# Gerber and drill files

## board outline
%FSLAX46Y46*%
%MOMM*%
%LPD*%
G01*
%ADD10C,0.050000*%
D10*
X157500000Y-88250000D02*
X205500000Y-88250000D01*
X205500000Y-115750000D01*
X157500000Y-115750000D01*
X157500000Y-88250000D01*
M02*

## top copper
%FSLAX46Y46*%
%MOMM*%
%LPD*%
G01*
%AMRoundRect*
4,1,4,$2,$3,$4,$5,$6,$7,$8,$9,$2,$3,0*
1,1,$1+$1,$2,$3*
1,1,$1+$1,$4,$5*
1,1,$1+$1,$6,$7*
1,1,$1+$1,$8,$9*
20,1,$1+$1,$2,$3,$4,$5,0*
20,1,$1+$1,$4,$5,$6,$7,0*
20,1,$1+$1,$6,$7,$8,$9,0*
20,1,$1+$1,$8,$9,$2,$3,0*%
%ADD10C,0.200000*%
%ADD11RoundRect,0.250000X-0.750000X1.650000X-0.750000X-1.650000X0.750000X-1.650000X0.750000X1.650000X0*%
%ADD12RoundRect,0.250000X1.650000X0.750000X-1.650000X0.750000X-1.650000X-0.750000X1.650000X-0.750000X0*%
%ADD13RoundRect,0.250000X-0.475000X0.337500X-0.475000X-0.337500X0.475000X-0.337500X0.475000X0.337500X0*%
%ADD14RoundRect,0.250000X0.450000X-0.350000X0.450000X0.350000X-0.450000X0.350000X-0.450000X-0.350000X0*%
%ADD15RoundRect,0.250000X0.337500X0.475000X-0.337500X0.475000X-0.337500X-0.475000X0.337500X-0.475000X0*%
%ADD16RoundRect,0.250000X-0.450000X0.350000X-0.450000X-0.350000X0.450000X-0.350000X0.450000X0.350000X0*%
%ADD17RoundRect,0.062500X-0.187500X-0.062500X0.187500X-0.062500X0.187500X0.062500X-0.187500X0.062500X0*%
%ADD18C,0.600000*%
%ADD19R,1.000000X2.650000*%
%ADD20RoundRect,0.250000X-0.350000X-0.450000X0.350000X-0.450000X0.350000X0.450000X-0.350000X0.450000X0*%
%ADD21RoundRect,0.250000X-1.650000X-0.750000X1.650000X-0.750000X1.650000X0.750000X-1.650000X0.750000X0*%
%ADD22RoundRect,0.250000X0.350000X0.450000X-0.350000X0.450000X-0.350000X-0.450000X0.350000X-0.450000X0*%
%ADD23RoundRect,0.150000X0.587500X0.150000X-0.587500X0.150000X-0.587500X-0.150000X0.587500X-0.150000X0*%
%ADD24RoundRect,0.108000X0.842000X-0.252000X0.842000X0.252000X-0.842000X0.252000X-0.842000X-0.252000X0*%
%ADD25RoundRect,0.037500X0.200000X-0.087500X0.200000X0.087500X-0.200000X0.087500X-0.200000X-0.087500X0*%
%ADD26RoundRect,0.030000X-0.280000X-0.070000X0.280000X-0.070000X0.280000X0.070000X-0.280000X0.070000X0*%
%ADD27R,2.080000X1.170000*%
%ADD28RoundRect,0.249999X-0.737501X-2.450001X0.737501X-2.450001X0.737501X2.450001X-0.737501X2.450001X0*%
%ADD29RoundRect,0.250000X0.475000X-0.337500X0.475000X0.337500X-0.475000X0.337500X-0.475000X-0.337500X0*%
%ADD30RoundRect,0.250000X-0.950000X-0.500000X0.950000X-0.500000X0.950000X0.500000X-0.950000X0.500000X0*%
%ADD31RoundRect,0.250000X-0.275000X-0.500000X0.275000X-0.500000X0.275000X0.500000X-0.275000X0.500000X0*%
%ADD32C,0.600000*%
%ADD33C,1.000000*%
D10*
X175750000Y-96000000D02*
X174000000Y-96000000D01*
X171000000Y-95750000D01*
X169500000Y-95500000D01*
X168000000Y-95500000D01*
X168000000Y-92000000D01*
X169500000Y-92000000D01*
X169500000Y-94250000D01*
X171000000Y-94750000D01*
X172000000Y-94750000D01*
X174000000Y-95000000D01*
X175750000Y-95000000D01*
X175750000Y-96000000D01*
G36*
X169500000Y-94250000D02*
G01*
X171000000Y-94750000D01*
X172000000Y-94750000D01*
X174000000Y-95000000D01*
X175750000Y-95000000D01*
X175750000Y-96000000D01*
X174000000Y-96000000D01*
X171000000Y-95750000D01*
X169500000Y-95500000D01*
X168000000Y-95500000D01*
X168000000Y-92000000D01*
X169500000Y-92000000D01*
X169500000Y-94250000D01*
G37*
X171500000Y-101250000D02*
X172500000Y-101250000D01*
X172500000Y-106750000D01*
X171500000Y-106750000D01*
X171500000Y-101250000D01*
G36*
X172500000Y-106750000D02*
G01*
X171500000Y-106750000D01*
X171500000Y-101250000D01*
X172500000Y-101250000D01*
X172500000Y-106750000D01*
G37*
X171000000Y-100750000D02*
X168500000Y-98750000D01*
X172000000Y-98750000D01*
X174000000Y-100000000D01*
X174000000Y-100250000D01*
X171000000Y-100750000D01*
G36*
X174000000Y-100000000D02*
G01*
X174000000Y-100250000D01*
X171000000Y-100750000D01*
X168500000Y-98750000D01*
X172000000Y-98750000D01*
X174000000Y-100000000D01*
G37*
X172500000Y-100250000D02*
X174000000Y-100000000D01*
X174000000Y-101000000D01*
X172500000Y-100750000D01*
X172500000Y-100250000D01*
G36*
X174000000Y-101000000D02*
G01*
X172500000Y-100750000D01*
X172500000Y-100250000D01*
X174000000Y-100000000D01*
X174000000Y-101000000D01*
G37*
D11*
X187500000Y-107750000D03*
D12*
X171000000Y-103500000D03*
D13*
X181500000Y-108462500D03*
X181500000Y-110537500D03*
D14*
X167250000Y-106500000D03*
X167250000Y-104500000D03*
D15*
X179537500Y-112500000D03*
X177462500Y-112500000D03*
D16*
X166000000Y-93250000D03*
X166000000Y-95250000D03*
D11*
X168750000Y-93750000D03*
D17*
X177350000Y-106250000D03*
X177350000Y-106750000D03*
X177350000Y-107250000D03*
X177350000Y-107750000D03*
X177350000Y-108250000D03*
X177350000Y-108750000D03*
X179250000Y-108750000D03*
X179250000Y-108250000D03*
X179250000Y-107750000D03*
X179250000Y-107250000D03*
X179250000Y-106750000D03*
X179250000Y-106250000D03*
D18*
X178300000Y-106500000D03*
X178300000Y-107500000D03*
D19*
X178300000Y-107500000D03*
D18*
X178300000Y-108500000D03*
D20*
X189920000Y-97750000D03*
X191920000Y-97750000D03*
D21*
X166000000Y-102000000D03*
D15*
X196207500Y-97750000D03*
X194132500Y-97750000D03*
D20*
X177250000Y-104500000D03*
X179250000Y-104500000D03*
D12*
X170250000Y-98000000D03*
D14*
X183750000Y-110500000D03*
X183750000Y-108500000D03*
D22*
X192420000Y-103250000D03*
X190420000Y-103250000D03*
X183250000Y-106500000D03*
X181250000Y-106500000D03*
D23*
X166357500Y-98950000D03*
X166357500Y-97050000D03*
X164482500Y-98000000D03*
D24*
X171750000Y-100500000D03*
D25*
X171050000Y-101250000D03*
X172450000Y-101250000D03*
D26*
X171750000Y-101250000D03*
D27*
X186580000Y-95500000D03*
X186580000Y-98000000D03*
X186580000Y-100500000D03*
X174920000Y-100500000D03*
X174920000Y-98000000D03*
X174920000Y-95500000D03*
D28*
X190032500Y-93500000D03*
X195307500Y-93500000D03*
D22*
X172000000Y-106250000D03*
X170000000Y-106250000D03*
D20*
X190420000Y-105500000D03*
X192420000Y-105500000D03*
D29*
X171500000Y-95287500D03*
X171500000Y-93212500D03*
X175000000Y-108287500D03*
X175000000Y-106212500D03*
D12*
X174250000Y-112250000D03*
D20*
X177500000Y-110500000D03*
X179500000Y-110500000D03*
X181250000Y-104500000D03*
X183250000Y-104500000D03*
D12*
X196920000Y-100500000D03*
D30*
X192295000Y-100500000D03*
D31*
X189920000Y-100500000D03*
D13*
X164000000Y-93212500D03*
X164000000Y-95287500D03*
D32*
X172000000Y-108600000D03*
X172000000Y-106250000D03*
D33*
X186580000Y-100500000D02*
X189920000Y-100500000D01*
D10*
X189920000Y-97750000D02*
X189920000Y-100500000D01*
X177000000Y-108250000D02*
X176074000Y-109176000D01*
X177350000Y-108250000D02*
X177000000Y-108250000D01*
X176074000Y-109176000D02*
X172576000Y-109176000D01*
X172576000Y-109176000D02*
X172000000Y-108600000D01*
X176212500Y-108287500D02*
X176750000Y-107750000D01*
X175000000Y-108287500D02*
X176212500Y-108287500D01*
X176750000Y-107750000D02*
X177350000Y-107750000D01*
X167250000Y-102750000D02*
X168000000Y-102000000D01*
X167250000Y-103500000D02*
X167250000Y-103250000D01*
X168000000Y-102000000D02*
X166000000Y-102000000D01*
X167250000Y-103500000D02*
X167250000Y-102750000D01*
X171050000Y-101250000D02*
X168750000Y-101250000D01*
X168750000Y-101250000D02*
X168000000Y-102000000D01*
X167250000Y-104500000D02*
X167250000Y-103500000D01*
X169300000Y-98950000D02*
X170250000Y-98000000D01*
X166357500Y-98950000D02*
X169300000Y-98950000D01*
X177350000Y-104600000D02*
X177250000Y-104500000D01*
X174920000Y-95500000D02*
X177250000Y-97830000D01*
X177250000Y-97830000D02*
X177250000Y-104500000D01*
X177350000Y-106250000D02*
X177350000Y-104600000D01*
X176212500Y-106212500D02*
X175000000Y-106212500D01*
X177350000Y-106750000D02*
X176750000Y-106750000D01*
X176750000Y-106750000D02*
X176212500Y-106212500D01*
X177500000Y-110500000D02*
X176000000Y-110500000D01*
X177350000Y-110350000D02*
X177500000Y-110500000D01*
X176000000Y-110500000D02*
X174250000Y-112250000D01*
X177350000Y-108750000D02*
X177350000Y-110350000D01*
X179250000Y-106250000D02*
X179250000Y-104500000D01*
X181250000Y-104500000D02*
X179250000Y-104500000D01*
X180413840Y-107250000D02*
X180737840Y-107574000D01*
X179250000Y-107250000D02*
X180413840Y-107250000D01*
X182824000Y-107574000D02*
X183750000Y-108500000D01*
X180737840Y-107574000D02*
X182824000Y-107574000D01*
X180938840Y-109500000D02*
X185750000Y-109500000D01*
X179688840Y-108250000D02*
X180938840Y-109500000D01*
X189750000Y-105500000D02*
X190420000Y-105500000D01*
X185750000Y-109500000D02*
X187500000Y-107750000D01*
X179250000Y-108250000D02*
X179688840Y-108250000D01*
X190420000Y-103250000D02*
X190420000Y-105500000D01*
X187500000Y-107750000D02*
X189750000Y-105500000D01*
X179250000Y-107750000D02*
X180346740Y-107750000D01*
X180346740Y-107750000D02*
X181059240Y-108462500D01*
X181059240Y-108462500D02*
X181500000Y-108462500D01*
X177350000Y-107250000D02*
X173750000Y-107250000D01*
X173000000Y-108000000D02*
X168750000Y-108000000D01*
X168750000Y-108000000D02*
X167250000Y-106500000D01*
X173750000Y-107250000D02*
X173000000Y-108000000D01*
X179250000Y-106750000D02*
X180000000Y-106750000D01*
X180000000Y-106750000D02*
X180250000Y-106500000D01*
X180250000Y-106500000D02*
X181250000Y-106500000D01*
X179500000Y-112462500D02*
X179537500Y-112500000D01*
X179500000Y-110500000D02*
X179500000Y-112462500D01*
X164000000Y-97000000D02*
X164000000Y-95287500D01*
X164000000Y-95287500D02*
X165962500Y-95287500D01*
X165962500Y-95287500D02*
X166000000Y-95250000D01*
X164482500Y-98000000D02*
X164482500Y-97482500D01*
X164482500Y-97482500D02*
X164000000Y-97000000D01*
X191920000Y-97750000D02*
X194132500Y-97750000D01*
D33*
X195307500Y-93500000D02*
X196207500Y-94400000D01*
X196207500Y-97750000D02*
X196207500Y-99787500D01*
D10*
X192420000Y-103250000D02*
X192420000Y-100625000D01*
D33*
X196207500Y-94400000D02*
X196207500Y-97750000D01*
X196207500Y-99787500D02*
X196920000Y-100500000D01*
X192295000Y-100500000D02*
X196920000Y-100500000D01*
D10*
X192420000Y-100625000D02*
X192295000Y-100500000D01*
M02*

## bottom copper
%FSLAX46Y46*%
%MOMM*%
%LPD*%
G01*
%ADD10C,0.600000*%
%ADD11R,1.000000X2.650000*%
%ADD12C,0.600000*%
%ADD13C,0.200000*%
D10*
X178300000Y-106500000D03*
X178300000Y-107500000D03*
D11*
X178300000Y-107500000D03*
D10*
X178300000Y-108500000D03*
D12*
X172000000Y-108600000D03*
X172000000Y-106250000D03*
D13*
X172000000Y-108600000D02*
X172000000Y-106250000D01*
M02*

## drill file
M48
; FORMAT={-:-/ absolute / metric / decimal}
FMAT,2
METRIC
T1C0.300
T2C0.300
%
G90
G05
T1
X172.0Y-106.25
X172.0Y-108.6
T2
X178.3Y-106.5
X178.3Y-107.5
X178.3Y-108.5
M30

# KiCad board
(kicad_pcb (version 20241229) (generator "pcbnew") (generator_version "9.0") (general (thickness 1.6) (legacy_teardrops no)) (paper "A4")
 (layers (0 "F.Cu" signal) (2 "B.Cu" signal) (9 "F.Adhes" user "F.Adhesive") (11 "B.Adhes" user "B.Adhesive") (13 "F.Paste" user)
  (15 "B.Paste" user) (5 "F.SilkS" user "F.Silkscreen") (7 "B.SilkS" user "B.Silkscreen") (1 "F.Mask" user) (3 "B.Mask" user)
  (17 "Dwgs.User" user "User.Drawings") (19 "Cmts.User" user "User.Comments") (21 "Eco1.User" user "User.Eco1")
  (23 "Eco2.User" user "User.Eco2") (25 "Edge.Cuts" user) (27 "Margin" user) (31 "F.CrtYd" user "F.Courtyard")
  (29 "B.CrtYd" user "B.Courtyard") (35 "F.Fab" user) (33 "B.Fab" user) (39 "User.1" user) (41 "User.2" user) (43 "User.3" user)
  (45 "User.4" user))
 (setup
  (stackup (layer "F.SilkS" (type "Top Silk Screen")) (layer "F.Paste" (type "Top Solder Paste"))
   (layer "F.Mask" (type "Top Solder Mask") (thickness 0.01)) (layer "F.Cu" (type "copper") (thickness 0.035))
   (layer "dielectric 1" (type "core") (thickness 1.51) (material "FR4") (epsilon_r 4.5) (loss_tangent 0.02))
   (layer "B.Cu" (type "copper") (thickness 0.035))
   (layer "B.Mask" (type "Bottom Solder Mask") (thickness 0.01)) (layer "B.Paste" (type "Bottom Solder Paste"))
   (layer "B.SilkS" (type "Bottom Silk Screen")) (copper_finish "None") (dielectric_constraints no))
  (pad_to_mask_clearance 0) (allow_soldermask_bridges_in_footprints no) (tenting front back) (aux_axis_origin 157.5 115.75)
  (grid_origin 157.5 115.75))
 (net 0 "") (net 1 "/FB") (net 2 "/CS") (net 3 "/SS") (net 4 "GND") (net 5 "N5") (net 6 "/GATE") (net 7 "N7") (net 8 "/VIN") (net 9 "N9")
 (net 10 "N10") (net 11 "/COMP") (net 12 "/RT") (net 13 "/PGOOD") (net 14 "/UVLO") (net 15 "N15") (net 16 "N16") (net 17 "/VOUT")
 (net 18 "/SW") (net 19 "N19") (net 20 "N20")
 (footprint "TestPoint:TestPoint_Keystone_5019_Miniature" (layer "F.Cu") (at 187.5 107.75 -90)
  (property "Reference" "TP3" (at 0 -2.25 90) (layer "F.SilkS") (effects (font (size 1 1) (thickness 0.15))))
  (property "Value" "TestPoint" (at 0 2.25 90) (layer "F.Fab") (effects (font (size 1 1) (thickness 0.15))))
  (pad "1" smd roundrect (at 0 0 270) (size 3.8 2) (layers "F.Cu" "F.Mask" "F.Paste") (roundrect_rratio 0.125) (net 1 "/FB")))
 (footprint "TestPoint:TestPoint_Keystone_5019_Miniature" (layer "F.Cu") (at 171 103.5 180)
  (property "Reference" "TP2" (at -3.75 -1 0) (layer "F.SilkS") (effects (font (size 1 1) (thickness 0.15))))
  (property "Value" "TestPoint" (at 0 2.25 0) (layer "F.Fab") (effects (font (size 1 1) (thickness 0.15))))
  (pad "1" smd roundrect (at 0 0 180) (size 3.8 2) (layers "F.Cu" "F.Mask" "F.Paste") (roundrect_rratio 0.125) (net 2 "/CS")))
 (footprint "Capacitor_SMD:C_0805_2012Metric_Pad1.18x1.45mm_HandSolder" (layer "F.Cu") (at 181.5 109.5 -90)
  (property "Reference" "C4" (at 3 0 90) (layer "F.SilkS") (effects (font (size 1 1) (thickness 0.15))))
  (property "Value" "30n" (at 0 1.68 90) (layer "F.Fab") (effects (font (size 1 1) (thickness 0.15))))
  (pad "1" smd roundrect (at -1.0375 0 270) (size 1.175 1.45) (layers "F.Cu" "F.Mask" "F.Paste") (roundrect_rratio 0.212766) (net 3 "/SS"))
  (pad "2" smd roundrect (at 1.0375 0 270) (size 1.175 1.45) (layers "F.Cu" "F.Mask" "F.Paste") (roundrect_rratio 0.212766) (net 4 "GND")))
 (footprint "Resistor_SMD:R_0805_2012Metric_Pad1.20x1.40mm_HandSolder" (layer "F.Cu") (at 167.25 105.5 90)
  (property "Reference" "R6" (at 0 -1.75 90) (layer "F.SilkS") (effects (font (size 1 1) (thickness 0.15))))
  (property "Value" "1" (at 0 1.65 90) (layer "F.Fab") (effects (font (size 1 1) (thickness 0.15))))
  (pad "1" smd roundrect (at -1 0 90) (size 1.2 1.4) (layers "F.Cu" "F.Mask" "F.Paste") (roundrect_rratio 0.208333) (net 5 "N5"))
  (pad "2" smd roundrect (at 1 0 90) (size 1.2 1.4) (layers "F.Cu" "F.Mask" "F.Paste") (roundrect_rratio 0.208333) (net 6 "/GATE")))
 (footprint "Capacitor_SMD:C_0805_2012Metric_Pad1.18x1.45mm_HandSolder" (layer "F.Cu") (at 178.5 112.5 180)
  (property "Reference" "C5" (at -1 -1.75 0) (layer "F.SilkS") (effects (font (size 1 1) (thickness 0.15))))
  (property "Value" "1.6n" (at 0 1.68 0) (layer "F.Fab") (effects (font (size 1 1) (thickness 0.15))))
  (pad "1" smd roundrect (at -1.0375 0 180) (size 1.175 1.45) (layers "F.Cu" "F.Mask" "F.Paste") (roundrect_rratio 0.212766) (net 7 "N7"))
  (pad "2" smd roundrect (at 1.0375 0 180) (size 1.175 1.45) (layers "F.Cu" "F.Mask" "F.Paste") (roundrect_rratio 0.212766) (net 4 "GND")))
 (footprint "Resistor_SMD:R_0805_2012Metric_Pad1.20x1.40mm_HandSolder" (layer "F.Cu") (at 166 94.25 -90)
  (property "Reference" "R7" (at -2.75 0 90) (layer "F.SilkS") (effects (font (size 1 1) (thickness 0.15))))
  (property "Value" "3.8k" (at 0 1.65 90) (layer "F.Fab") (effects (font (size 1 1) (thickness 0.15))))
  (pad "1" smd roundrect (at -1 0 270) (size 1.2 1.4) (layers "F.Cu" "F.Mask" "F.Paste") (roundrect_rratio 0.208333) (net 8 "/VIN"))
  (pad "2" smd roundrect (at 1 0 270) (size 1.2 1.4) (layers "F.Cu" "F.Mask" "F.Paste") (roundrect_rratio 0.208333) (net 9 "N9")))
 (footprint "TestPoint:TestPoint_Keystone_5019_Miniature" (layer "F.Cu") (at 168.75 93.75 -90)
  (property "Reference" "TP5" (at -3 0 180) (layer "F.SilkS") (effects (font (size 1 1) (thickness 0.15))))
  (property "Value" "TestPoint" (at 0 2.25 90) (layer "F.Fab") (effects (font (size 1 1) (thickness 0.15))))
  (pad "1" smd roundrect (at 0 0 270) (size 3.8 2) (layers "F.Cu" "F.Mask" "F.Paste") (roundrect_rratio 0.125) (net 8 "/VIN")))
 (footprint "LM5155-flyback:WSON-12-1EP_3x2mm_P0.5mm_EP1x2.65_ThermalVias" (layer "F.Cu") (at 178.3 107.5)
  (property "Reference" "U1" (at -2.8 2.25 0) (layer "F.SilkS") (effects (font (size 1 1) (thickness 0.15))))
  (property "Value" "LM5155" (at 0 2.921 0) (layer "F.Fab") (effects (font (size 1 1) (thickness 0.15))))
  (pad "" smd rect (at 0 -0.5) (size 0.95 0.8) (layers "F.Paste"))
  (pad "" smd rect (at 0 0.5) (size 0.95 0.8) (layers "F.Paste"))
  (pad "1" smd roundrect (at -0.95 -1.25) (size 0.5 0.25) (layers "F.Cu" "F.Mask" "F.Paste") (roundrect_rratio 0.25) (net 8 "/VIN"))
  (pad "2" smd roundrect (at -0.95 -0.75) (size 0.5 0.25) (layers "F.Cu" "F.Mask" "F.Paste") (roundrect_rratio 0.25) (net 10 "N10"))
  (pad "3" smd roundrect (at -0.95 -0.25) (size 0.5 0.25) (layers "F.Cu" "F.Mask" "F.Paste") (roundrect_rratio 0.25) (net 5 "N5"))
  (pad "4" smd roundrect (at -0.95 0.25) (size 0.5 0.25) (layers "F.Cu" "F.Mask" "F.Paste") (roundrect_rratio 0.25) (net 4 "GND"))
  (pad "5" smd roundrect (at -0.95 0.75) (size 0.5 0.25) (layers "F.Cu" "F.Mask" "F.Paste") (roundrect_rratio 0.25) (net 2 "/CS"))
  (pad "6" smd roundrect (at -0.95 1.25) (size 0.5 0.25) (layers "F.Cu" "F.Mask" "F.Paste") (roundrect_rratio 0.25) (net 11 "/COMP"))
  (pad "7" smd roundrect (at 0.95 1.25) (size 0.5 0.25) (layers "F.Cu" "F.Mask" "F.Paste") (roundrect_rratio 0.25) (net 4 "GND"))
  (pad "8" smd roundrect (at 0.95 0.75) (size 0.5 0.25) (layers "F.Cu" "F.Mask" "F.Paste") (roundrect_rratio 0.25) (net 1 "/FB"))
  (pad "9" smd roundrect (at 0.95 0.25) (size 0.5 0.25) (layers "F.Cu" "F.Mask" "F.Paste") (roundrect_rratio 0.25) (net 3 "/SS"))
  (pad "10" smd roundrect (at 0.95 -0.25) (size 0.5 0.25) (layers "F.Cu" "F.Mask" "F.Paste") (roundrect_rratio 0.25) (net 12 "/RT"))
  (pad "11" smd roundrect (at 0.95 -0.75) (size 0.5 0.25) (layers "F.Cu" "F.Mask" "F.Paste") (roundrect_rratio 0.25) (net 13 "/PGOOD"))
  (pad "12" smd roundrect (at 0.95 -1.25) (size 0.5 0.25) (layers "F.Cu" "F.Mask" "F.Paste") (roundrect_rratio 0.25) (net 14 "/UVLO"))
  (pad "13" thru_hole circle (at 0 -1 90) (size 0.6 0.6) (drill 0.3) (layers "*.Cu") (remove_unused_layers no) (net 4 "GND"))
  (pad "13" thru_hole circle (at 0 0) (size 0.6 0.6) (drill 0.3) (layers "*.Cu") (remove_unused_layers no) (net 4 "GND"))
  (pad "13" smd rect (at 0 0) (size 1 2.65) (layers "F.Cu" "F.Mask") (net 4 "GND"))
  (pad "13" smd rect (at 0 0) (size 1 2.65) (layers "B.Cu") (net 4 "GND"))
  (pad "13" thru_hole circle (at 0 1) (size 0.6 0.6) (drill 0.3) (layers "*.Cu") (remove_unused_layers no) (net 4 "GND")))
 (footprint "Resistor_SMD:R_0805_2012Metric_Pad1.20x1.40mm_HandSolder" (layer "F.Cu") (at 190.92 97.75)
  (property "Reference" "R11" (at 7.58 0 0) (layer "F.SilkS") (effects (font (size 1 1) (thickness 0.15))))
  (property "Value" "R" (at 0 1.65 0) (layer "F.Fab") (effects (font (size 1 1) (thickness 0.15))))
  (pad "1" smd roundrect (at -1 0) (size 1.2 1.4) (layers "F.Cu" "F.Mask" "F.Paste") (roundrect_rratio 0.208333) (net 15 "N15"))
  (pad "2" smd roundrect (at 1 0) (size 1.2 1.4) (layers "F.Cu" "F.Mask" "F.Paste") (roundrect_rratio 0.208333) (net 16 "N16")))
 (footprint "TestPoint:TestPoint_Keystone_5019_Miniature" (layer "F.Cu") (at 166 102)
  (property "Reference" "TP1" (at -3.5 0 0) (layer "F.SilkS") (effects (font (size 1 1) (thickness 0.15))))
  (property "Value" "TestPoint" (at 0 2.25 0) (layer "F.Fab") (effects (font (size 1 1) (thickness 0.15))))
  (pad "1" smd roundrect (at 0 0) (size 3.8 2) (layers "F.Cu" "F.Mask" "F.Paste") (roundrect_rratio 0.125) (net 6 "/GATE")))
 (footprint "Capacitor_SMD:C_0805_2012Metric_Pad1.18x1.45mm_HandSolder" (layer "F.Cu") (at 195.17 97.75 180)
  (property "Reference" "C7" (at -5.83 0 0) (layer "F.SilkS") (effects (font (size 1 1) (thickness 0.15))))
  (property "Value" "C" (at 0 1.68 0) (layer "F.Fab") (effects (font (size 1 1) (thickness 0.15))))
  (pad "1" smd roundrect (at -1.0375 0 180) (size 1.175 1.45) (layers "F.Cu" "F.Mask" "F.Paste") (roundrect_rratio 0.212766)
   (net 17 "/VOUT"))
  (pad "2" smd roundrect (at 1.0375 0 180) (size 1.175 1.45) (layers "F.Cu" "F.Mask" "F.Paste") (roundrect_rratio 0.212766) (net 16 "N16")))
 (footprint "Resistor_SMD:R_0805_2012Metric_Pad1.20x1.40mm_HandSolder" (layer "F.Cu") (at 178.25 104.5)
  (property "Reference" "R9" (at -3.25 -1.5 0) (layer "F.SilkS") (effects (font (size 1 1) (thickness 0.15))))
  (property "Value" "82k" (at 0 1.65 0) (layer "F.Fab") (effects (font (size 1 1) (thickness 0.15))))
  (pad "1" smd roundrect (at -1 0) (size 1.2 1.4) (layers "F.Cu" "F.Mask" "F.Paste") (roundrect_rratio 0.208333) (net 8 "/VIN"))
  (pad "2" smd roundrect (at 1 0) (size 1.2 1.4) (layers "F.Cu" "F.Mask" "F.Paste") (roundrect_rratio 0.208333) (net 14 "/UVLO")))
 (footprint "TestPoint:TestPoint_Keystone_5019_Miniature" (layer "F.Cu") (at 170.25 98 180)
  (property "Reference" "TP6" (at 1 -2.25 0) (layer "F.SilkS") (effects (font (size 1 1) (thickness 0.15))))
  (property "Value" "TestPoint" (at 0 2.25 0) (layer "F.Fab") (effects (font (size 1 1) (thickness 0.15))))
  (pad "1" smd roundrect (at 0 0 180) (size 3.8 2) (layers "F.Cu" "F.Mask" "F.Paste") (roundrect_rratio 0.125) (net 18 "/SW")))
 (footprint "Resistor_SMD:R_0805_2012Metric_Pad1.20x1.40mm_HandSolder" (layer "F.Cu") (at 183.75 109.5 90)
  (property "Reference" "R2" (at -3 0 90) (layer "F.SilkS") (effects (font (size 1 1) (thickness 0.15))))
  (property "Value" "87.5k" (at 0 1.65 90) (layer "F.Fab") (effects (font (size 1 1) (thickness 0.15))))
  (pad "1" smd roundrect (at -1 0 90) (size 1.2 1.4) (layers "F.Cu" "F.Mask" "F.Paste") (roundrect_rratio 0.208333) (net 4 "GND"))
  (pad "2" smd roundrect (at 1 0 90) (size 1.2 1.4) (layers "F.Cu" "F.Mask" "F.Paste") (roundrect_rratio 0.208333) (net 12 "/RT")))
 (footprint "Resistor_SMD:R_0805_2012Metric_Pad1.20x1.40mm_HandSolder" (layer "F.Cu") (at 191.42 103.25 180)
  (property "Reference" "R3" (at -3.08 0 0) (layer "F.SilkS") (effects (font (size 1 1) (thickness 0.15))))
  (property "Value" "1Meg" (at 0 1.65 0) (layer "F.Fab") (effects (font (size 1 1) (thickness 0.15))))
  (pad "1" smd roundrect (at -1 0 180) (size 1.2 1.4) (layers "F.Cu" "F.Mask" "F.Paste") (roundrect_rratio 0.208333) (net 17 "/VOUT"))
  (pad "2" smd roundrect (at 1 0 180) (size 1.2 1.4) (layers "F.Cu" "F.Mask" "F.Paste") (roundrect_rratio 0.208333) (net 1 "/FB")))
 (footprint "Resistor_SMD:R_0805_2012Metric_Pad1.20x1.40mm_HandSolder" (layer "F.Cu") (at 182.25 106.5 180)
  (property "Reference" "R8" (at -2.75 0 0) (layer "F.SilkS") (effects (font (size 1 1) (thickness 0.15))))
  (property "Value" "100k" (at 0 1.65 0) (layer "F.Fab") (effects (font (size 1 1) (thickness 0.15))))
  (pad "1" smd roundrect (at -1 0 180) (size 1.2 1.4) (layers "F.Cu" "F.Mask" "F.Paste") (roundrect_rratio 0.208333) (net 8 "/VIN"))
  (pad "2" smd roundrect (at 1 0 180) (size 1.2 1.4) (layers "F.Cu" "F.Mask" "F.Paste") (roundrect_rratio 0.208333) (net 13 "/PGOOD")))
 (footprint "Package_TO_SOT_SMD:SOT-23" (layer "F.Cu") (at 165.42 98 180)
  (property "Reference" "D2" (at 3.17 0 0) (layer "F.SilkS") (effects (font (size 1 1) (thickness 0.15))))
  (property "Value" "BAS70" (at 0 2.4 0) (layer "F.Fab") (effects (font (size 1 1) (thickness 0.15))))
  (pad "1" smd roundrect (at -0.9375 -0.95 180) (size 1.475 0.6) (layers "F.Cu" "F.Mask" "F.Paste") (roundrect_rratio 0.25) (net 18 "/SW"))
  (pad "2" smd roundrect (at -0.9375 0.95 180) (size 1.475 0.6) (layers "F.Cu" "F.Mask" "F.Paste") (roundrect_rratio 0.25) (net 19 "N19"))
  (pad "3" smd roundrect (at 0.9375 0 180) (size 1.475 0.6) (layers "F.Cu" "F.Mask" "F.Paste") (roundrect_rratio 0.25) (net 9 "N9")))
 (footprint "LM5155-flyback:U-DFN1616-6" (layer "F.Cu") (at 171.75 100.75 -90)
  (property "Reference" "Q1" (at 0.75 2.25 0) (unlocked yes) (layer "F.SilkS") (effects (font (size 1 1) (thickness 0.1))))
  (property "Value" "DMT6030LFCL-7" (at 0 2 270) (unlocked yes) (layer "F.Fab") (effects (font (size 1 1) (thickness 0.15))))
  (pad "1" smd roundrect (at -0.25 0 90) (size 0.72 1.9) (layers "F.Cu" "F.Mask" "F.Paste") (roundrect_rratio 0.15) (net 18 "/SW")
   (thermal_bridge_angle 45))
  (pad "2" smd roundrect (at 0.5 0.7 90) (size 0.25 0.475) (layers "F.Cu" "F.Mask" "F.Paste") (roundrect_rratio 0.15) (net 6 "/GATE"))
  (pad "3" smd roundrect (at 0.5 -0.7 90) (size 0.25 0.475) (layers "F.Cu" "F.Mask" "F.Paste") (roundrect_rratio 0.15) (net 2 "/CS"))
  (pad "3" smd roundrect (at 0.5 0) (size 0.62 0.2) (layers "F.Cu" "F.Mask" "F.Paste") (roundrect_rratio 0.15) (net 2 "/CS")))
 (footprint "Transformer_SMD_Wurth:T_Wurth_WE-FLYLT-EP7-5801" (layer "F.Cu") (at 180.75 98 -90)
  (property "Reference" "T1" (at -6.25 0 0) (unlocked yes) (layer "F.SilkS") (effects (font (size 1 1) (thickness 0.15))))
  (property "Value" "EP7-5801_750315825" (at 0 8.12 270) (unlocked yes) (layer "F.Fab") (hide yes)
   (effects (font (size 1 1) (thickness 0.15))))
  (pad "1" smd rect (at -2.5 -5.83 270) (size 1.17 2.08) (layers "F.Cu" "F.Mask" "F.Paste") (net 4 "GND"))
  (pad "2" smd rect (at 0 -5.83 270) (size 1.17 2.08) (layers "F.Cu" "F.Mask" "F.Paste") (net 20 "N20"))
  (pad "3" smd rect (at 2.5 -5.83 270) (size 1.17 2.08) (layers "F.Cu" "F.Mask" "F.Paste") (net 15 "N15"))
  (pad "4" smd rect (at 2.5 5.83 270) (size 1.17 2.08) (layers "F.Cu" "F.Mask" "F.Paste") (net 18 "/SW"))
  (pad "5" smd rect (at 0 5.83 270) (size 1.17 2.08) (layers "F.Cu" "F.Mask" "F.Paste"))
  (pad "6" smd rect (at -2.5 5.83 270) (size 1.17 2.08) (layers "F.Cu" "F.Mask" "F.Paste") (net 8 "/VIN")))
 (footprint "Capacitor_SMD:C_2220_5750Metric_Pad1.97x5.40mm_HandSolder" (layer "F.Cu") (at 192.67 93.5)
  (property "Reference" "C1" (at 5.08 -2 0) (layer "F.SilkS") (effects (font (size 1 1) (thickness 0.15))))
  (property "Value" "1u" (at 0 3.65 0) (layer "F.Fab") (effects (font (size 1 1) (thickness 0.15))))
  (pad "1" smd roundrect (at -2.6375 0) (size 1.975 5.4) (layers "F.Cu" "F.Mask" "F.Paste") (roundrect_rratio 0.126582) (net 4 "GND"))
  (pad "2" smd roundrect (at 2.6375 0) (size 1.975 5.4) (layers "F.Cu" "F.Mask" "F.Paste") (roundrect_rratio 0.126582) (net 17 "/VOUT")))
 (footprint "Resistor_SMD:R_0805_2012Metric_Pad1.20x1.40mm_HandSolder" (layer "F.Cu") (at 171 106.25 180)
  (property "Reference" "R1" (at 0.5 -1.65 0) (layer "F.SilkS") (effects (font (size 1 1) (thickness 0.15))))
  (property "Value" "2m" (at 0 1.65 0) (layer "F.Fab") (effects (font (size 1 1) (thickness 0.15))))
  (pad "1" smd roundrect (at -1 0 180) (size 1.2 1.4) (layers "F.Cu" "F.Mask" "F.Paste") (roundrect_rratio 0.208333) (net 2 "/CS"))
  (pad "2" smd roundrect (at 1 0 180) (size 1.2 1.4) (layers "F.Cu" "F.Mask" "F.Paste") (roundrect_rratio 0.208333) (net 4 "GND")))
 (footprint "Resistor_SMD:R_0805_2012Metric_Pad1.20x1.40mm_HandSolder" (layer "F.Cu") (at 191.42 105.5)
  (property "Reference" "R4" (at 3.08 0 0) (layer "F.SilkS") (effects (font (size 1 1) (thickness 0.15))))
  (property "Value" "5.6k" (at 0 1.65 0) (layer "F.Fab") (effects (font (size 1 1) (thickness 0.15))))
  (pad "1" smd roundrect (at -1 0) (size 1.2 1.4) (layers "F.Cu" "F.Mask" "F.Paste") (roundrect_rratio 0.208333) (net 1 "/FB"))
  (pad "2" smd roundrect (at 1 0) (size 1.2 1.4) (layers "F.Cu" "F.Mask" "F.Paste") (roundrect_rratio 0.208333) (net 4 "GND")))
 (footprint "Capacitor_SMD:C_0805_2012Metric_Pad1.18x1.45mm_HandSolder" (layer "F.Cu") (at 171.5 94.25 90)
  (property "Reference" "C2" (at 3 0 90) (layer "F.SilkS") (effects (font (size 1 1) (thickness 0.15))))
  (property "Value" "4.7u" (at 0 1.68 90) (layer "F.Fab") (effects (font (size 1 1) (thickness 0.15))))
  (pad "1" smd roundrect (at -1.0375 0 90) (size 1.175 1.45) (layers "F.Cu" "F.Mask" "F.Paste") (roundrect_rratio 0.212766) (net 8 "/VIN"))
  (pad "2" smd roundrect (at 1.0375 0 90) (size 1.175 1.45) (layers "F.Cu" "F.Mask" "F.Paste") (roundrect_rratio 0.212766) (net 4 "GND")))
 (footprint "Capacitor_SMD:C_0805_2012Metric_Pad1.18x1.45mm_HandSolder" (layer "F.Cu") (at 175 107.25 90)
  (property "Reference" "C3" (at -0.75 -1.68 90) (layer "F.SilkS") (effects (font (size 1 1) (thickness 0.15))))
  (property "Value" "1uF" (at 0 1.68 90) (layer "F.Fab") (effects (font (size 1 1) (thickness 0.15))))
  (pad "1" smd roundrect (at -1.0375 0 90) (size 1.175 1.45) (layers "F.Cu" "F.Mask" "F.Paste") (roundrect_rratio 0.212766) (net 4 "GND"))
  (pad "2" smd roundrect (at 1.0375 0 90) (size 1.175 1.45) (layers "F.Cu" "F.Mask" "F.Paste") (roundrect_rratio 0.212766) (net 10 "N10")))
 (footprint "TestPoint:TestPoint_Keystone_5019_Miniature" (layer "F.Cu") (at 174.25 112.25 180)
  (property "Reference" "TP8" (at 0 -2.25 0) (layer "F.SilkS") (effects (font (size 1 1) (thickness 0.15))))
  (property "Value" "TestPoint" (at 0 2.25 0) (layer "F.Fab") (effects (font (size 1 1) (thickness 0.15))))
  (pad "1" smd roundrect (at 0 0 180) (size 3.8 2) (layers "F.Cu" "F.Mask" "F.Paste") (roundrect_rratio 0.125) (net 11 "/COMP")))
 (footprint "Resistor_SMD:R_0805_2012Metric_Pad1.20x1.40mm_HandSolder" (layer "F.Cu") (at 178.5 110.5)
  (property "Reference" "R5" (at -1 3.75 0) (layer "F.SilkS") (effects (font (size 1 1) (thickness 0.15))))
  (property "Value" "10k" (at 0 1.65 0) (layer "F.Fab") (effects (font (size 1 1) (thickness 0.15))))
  (pad "1" smd roundrect (at -1 0) (size 1.2 1.4) (layers "F.Cu" "F.Mask" "F.Paste") (roundrect_rratio 0.208333) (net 11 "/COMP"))
  (pad "2" smd roundrect (at 1 0) (size 1.2 1.4) (layers "F.Cu" "F.Mask" "F.Paste") (roundrect_rratio 0.208333) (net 7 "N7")))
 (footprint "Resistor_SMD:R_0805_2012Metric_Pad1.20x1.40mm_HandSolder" (layer "F.Cu") (at 182.25 104.5)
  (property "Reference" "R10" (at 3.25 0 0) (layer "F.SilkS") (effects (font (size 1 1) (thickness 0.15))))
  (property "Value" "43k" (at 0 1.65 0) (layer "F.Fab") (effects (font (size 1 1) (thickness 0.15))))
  (pad "1" smd roundrect (at -1 0) (size 1.2 1.4) (layers "F.Cu" "F.Mask" "F.Paste") (roundrect_rratio 0.208333) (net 14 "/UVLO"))
  (pad "2" smd roundrect (at 1 0) (size 1.2 1.4) (layers "F.Cu" "F.Mask" "F.Paste") (roundrect_rratio 0.208333) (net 4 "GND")))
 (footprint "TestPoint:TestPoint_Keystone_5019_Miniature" (layer "F.Cu") (at 196.92 100.5 180)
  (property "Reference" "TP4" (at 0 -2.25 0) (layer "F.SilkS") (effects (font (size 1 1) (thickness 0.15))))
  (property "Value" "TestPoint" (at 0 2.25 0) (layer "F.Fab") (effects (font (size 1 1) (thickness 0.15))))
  (pad "1" smd roundrect (at 0 0 180) (size 3.8 2) (layers "F.Cu" "F.Mask" "F.Paste") (roundrect_rratio 0.125) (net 17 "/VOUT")))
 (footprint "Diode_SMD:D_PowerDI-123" (layer "F.Cu") (at 191.445 100.5 180)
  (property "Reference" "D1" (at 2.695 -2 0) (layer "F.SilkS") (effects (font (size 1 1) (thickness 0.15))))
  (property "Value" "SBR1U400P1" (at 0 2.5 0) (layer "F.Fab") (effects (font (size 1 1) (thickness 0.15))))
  (pad "1" smd roundrect (at -0.85 0) (size 2.4 1.5) (layers "F.Cu" "F.Mask" "F.Paste") (roundrect_rratio 0.1666666667) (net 17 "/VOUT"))
  (pad "2" smd roundrect (at 1.525 0) (size 1.05 1.5) (layers "F.Cu" "F.Mask" "F.Paste") (roundrect_rratio 0.2380952381) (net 15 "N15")))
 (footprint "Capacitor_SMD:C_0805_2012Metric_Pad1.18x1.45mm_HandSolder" (layer "F.Cu") (at 164 94.25 -90)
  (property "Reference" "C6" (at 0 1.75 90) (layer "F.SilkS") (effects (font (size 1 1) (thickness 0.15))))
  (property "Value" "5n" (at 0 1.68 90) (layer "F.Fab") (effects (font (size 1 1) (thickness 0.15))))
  (pad "1" smd roundrect (at -1.0375 0 270) (size 1.175 1.45) (layers "F.Cu" "F.Mask" "F.Paste") (roundrect_rratio 0.212766) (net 8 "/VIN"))
  (pad "2" smd roundrect (at 1.0375 0 270) (size 1.175 1.45) (layers "F.Cu" "F.Mask" "F.Paste") (roundrect_rratio 0.212766) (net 9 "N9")))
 (gr_poly
  (pts (xy 175.75 96) (xy 174 96) (xy 171 95.75) (xy 169.5 95.5) (xy 168 95.5) (xy 168 92) (xy 169.5 92) (xy 169.5 94.25) (xy 171 94.75)
   (xy 172 94.75) (xy 174 95) (xy 175.75 95))
  (stroke (width 0.2) (type solid)) (fill yes) (layer "F.Cu") (net 8))
 (gr_poly
  (pts (xy 171.5 101.25) (xy 172.5 101.25) (xy 172.5 106.75) (xy 171.5 106.75)) (stroke (width 0.2) (type solid)) (fill yes) (layer "F.Cu")
  (net 2))
 (gr_poly
  (pts (xy 171 100.75) (xy 168.5 98.75) (xy 172 98.75) (xy 174 100) (xy 174 100.25)) (stroke (width 0.2) (type solid)) (fill yes)
  (layer "F.Cu") (net 18))
 (gr_poly
  (pts (xy 172.5 100.25) (xy 174 100) (xy 174 101) (xy 172.5 100.75)) (stroke (width 0.2) (type solid)) (fill yes) (layer "F.Cu") (net 18))
 (gr_rect (start 157.5 88.25) (end 205.5 115.75) (stroke (width 0.05) (type default)) (fill no) (layer "Edge.Cuts"))
 (segment (start 186.58 100.5) (end 189.92 100.5) (width 1) (layer "F.Cu") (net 15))
 (segment (start 189.92 97.75) (end 189.92 100.5) (width 0.2) (layer "F.Cu") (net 15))
 (segment (start 177 108.25) (end 176.074 109.176) (width 0.2) (layer "F.Cu") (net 2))
 (segment (start 177.35 108.25) (end 177 108.25) (width 0.2) (layer "F.Cu") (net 2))
 (segment (start 176.074 109.176) (end 172.576 109.176) (width 0.2) (layer "F.Cu") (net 2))
 (segment (start 172.576 109.176) (end 172 108.6) (width 0.2) (layer "F.Cu") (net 2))
 (via (at 172 108.6) (size 0.6) (drill 0.3) (layers "F.Cu" "B.Cu") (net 2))
 (via (at 172 106.25) (size 0.6) (drill 0.3) (layers "F.Cu" "B.Cu") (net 2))
 (segment (start 172 108.6) (end 172 106.25) (width 0.2) (layer "B.Cu") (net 2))
 (segment (start 176.2125 108.2875) (end 176.75 107.75) (width 0.2) (layer "F.Cu") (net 4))
 (segment (start 175 108.2875) (end 176.2125 108.2875) (width 0.2) (layer "F.Cu") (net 4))
 (segment (start 176.75 107.75) (end 177.35 107.75) (width 0.2) (layer "F.Cu") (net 4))
 (segment (start 167.25 102.75) (end 168 102) (width 0.2) (layer "F.Cu") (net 6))
 (segment (start 167.25 103.5) (end 167.25 103.25) (width 0.2) (layer "F.Cu") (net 6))
 (segment (start 168 102) (end 166 102) (width 0.2) (layer "F.Cu") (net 6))
 (segment (start 167.25 103.5) (end 167.25 102.75) (width 0.2) (layer "F.Cu") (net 6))
 (segment (start 171.05 101.25) (end 168.75 101.25) (width 0.2) (layer "F.Cu") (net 6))
 (segment (start 168.75 101.25) (end 168 102) (width 0.2) (layer "F.Cu") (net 6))
 (segment (start 167.25 104.5) (end 167.25 103.5) (width 0.2) (layer "F.Cu") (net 6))
 (segment (start 169.3 98.95) (end 170.25 98) (width 0.2) (layer "F.Cu") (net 18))
 (segment (start 166.3575 98.95) (end 169.3 98.95) (width 0.2) (layer "F.Cu") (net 18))
 (segment (start 177.35 104.6) (end 177.25 104.5) (width 0.2) (layer "F.Cu") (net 8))
 (segment (start 174.92 95.5) (end 177.25 97.83) (width 0.2) (layer "F.Cu") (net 8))
 (segment (start 177.25 97.83) (end 177.25 104.5) (width 0.2) (layer "F.Cu") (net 8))
 (segment (start 177.35 106.25) (end 177.35 104.6) (width 0.2) (layer "F.Cu") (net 8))
 (segment (start 176.2125 106.2125) (end 175 106.2125) (width 0.2) (layer "F.Cu") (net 10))
 (segment (start 177.35 106.75) (end 176.75 106.75) (width 0.2) (layer "F.Cu") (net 10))
 (segment (start 176.75 106.75) (end 176.2125 106.2125) (width 0.2) (layer "F.Cu") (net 10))
 (segment (start 177.5 110.5) (end 176 110.5) (width 0.2) (layer "F.Cu") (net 11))
 (segment (start 177.35 110.35) (end 177.5 110.5) (width 0.2) (layer "F.Cu") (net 11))
 (segment (start 176 110.5) (end 174.25 112.25) (width 0.2) (layer "F.Cu") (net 11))
 (segment (start 177.35 108.75) (end 177.35 110.35) (width 0.2) (layer "F.Cu") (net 11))
 (segment (start 179.25 106.25) (end 179.25 104.5) (width 0.2) (layer "F.Cu") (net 14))
 (segment (start 181.25 104.5) (end 179.25 104.5) (width 0.2) (layer "F.Cu") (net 14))
 (segment (start 180.41384 107.25) (end 180.73784 107.574) (width 0.2) (layer "F.Cu") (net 12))
 (segment (start 179.25 107.25) (end 180.41384 107.25) (width 0.2) (layer "F.Cu") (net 12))
 (segment (start 182.824 107.574) (end 183.75 108.5) (width 0.2) (layer "F.Cu") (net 12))
 (segment (start 180.73784 107.574) (end 182.824 107.574) (width 0.2) (layer "F.Cu") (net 12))
 (segment (start 180.93884 109.5) (end 185.75 109.5) (width 0.2) (layer "F.Cu") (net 1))
 (segment (start 179.68884 108.25) (end 180.93884 109.5) (width 0.2) (layer "F.Cu") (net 1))
 (segment (start 189.75 105.5) (end 190.42 105.5) (width 0.2) (layer "F.Cu") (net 1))
 (segment (start 185.75 109.5) (end 187.5 107.75) (width 0.2) (layer "F.Cu") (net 1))
 (segment (start 179.25 108.25) (end 179.68884 108.25) (width 0.2) (layer "F.Cu") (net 1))
 (segment (start 190.42 103.25) (end 190.42 105.5) (width 0.2) (layer "F.Cu") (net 1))
 (segment (start 187.5 107.75) (end 189.75 105.5) (width 0.2) (layer "F.Cu") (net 1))
 (segment (start 179.25 107.75) (end 180.34674 107.75) (width 0.2) (layer "F.Cu") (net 3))
 (segment (start 180.34674 107.75) (end 181.05924 108.4625) (width 0.2) (layer "F.Cu") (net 3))
 (segment (start 181.05924 108.4625) (end 181.5 108.4625) (width 0.2) (layer "F.Cu") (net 3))
 (segment (start 177.35 107.25) (end 173.75 107.25) (width 0.2) (layer "F.Cu") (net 5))
 (segment (start 173 108) (end 168.75 108) (width 0.2) (layer "F.Cu") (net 5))
 (segment (start 168.75 108) (end 167.25 106.5) (width 0.2) (layer "F.Cu") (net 5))
 (segment (start 173.75 107.25) (end 173 108) (width 0.2) (layer "F.Cu") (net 5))
 (segment (start 179.25 106.75) (end 180 106.75) (width 0.2) (layer "F.Cu") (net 13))
 (segment (start 180 106.75) (end 180.25 106.5) (width 0.2) (layer "F.Cu") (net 13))
 (segment (start 180.25 106.5) (end 181.25 106.5) (width 0.2) (layer "F.Cu") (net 13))
 (segment (start 179.5 112.4625) (end 179.5375 112.5) (width 0.2) (layer "F.Cu") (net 7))
 (segment (start 179.5 110.5) (end 179.5 112.4625) (width 0.2) (layer "F.Cu") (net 7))
 (segment (start 164 97) (end 164 95.2875) (width 0.2) (layer "F.Cu") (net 9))
 (segment (start 164 95.2875) (end 165.9625 95.2875) (width 0.2) (layer "F.Cu") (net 9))
 (segment (start 165.9625 95.2875) (end 166 95.25) (width 0.2) (layer "F.Cu") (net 9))
 (segment (start 164.4825 98) (end 164.4825 97.4825) (width 0.2) (layer "F.Cu") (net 9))
 (segment (start 164.4825 97.4825) (end 164 97) (width 0.2) (layer "F.Cu") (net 9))
 (segment (start 191.92 97.75) (end 194.1325 97.75) (width 0.2) (layer "F.Cu") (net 16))
 (segment (start 195.3075 93.5) (end 196.2075 94.4) (width 1) (layer "F.Cu") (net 17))
 (segment (start 196.2075 97.75) (end 196.2075 99.7875) (width 1) (layer "F.Cu") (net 17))
 (segment (start 192.42 103.25) (end 192.42 100.625) (width 0.2) (layer "F.Cu") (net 17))
 (segment (start 196.2075 94.4) (end 196.2075 97.75) (width 1) (layer "F.Cu") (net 17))
 (segment (start 196.2075 99.7875) (end 196.92 100.5) (width 1) (layer "F.Cu") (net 17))
 (segment (start 192.295 100.5) (end 196.92 100.5) (width 1) (layer "F.Cu") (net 17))
 (segment (start 192.42 100.625) (end 192.295 100.5) (width 0.2) (layer "F.Cu") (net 17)))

